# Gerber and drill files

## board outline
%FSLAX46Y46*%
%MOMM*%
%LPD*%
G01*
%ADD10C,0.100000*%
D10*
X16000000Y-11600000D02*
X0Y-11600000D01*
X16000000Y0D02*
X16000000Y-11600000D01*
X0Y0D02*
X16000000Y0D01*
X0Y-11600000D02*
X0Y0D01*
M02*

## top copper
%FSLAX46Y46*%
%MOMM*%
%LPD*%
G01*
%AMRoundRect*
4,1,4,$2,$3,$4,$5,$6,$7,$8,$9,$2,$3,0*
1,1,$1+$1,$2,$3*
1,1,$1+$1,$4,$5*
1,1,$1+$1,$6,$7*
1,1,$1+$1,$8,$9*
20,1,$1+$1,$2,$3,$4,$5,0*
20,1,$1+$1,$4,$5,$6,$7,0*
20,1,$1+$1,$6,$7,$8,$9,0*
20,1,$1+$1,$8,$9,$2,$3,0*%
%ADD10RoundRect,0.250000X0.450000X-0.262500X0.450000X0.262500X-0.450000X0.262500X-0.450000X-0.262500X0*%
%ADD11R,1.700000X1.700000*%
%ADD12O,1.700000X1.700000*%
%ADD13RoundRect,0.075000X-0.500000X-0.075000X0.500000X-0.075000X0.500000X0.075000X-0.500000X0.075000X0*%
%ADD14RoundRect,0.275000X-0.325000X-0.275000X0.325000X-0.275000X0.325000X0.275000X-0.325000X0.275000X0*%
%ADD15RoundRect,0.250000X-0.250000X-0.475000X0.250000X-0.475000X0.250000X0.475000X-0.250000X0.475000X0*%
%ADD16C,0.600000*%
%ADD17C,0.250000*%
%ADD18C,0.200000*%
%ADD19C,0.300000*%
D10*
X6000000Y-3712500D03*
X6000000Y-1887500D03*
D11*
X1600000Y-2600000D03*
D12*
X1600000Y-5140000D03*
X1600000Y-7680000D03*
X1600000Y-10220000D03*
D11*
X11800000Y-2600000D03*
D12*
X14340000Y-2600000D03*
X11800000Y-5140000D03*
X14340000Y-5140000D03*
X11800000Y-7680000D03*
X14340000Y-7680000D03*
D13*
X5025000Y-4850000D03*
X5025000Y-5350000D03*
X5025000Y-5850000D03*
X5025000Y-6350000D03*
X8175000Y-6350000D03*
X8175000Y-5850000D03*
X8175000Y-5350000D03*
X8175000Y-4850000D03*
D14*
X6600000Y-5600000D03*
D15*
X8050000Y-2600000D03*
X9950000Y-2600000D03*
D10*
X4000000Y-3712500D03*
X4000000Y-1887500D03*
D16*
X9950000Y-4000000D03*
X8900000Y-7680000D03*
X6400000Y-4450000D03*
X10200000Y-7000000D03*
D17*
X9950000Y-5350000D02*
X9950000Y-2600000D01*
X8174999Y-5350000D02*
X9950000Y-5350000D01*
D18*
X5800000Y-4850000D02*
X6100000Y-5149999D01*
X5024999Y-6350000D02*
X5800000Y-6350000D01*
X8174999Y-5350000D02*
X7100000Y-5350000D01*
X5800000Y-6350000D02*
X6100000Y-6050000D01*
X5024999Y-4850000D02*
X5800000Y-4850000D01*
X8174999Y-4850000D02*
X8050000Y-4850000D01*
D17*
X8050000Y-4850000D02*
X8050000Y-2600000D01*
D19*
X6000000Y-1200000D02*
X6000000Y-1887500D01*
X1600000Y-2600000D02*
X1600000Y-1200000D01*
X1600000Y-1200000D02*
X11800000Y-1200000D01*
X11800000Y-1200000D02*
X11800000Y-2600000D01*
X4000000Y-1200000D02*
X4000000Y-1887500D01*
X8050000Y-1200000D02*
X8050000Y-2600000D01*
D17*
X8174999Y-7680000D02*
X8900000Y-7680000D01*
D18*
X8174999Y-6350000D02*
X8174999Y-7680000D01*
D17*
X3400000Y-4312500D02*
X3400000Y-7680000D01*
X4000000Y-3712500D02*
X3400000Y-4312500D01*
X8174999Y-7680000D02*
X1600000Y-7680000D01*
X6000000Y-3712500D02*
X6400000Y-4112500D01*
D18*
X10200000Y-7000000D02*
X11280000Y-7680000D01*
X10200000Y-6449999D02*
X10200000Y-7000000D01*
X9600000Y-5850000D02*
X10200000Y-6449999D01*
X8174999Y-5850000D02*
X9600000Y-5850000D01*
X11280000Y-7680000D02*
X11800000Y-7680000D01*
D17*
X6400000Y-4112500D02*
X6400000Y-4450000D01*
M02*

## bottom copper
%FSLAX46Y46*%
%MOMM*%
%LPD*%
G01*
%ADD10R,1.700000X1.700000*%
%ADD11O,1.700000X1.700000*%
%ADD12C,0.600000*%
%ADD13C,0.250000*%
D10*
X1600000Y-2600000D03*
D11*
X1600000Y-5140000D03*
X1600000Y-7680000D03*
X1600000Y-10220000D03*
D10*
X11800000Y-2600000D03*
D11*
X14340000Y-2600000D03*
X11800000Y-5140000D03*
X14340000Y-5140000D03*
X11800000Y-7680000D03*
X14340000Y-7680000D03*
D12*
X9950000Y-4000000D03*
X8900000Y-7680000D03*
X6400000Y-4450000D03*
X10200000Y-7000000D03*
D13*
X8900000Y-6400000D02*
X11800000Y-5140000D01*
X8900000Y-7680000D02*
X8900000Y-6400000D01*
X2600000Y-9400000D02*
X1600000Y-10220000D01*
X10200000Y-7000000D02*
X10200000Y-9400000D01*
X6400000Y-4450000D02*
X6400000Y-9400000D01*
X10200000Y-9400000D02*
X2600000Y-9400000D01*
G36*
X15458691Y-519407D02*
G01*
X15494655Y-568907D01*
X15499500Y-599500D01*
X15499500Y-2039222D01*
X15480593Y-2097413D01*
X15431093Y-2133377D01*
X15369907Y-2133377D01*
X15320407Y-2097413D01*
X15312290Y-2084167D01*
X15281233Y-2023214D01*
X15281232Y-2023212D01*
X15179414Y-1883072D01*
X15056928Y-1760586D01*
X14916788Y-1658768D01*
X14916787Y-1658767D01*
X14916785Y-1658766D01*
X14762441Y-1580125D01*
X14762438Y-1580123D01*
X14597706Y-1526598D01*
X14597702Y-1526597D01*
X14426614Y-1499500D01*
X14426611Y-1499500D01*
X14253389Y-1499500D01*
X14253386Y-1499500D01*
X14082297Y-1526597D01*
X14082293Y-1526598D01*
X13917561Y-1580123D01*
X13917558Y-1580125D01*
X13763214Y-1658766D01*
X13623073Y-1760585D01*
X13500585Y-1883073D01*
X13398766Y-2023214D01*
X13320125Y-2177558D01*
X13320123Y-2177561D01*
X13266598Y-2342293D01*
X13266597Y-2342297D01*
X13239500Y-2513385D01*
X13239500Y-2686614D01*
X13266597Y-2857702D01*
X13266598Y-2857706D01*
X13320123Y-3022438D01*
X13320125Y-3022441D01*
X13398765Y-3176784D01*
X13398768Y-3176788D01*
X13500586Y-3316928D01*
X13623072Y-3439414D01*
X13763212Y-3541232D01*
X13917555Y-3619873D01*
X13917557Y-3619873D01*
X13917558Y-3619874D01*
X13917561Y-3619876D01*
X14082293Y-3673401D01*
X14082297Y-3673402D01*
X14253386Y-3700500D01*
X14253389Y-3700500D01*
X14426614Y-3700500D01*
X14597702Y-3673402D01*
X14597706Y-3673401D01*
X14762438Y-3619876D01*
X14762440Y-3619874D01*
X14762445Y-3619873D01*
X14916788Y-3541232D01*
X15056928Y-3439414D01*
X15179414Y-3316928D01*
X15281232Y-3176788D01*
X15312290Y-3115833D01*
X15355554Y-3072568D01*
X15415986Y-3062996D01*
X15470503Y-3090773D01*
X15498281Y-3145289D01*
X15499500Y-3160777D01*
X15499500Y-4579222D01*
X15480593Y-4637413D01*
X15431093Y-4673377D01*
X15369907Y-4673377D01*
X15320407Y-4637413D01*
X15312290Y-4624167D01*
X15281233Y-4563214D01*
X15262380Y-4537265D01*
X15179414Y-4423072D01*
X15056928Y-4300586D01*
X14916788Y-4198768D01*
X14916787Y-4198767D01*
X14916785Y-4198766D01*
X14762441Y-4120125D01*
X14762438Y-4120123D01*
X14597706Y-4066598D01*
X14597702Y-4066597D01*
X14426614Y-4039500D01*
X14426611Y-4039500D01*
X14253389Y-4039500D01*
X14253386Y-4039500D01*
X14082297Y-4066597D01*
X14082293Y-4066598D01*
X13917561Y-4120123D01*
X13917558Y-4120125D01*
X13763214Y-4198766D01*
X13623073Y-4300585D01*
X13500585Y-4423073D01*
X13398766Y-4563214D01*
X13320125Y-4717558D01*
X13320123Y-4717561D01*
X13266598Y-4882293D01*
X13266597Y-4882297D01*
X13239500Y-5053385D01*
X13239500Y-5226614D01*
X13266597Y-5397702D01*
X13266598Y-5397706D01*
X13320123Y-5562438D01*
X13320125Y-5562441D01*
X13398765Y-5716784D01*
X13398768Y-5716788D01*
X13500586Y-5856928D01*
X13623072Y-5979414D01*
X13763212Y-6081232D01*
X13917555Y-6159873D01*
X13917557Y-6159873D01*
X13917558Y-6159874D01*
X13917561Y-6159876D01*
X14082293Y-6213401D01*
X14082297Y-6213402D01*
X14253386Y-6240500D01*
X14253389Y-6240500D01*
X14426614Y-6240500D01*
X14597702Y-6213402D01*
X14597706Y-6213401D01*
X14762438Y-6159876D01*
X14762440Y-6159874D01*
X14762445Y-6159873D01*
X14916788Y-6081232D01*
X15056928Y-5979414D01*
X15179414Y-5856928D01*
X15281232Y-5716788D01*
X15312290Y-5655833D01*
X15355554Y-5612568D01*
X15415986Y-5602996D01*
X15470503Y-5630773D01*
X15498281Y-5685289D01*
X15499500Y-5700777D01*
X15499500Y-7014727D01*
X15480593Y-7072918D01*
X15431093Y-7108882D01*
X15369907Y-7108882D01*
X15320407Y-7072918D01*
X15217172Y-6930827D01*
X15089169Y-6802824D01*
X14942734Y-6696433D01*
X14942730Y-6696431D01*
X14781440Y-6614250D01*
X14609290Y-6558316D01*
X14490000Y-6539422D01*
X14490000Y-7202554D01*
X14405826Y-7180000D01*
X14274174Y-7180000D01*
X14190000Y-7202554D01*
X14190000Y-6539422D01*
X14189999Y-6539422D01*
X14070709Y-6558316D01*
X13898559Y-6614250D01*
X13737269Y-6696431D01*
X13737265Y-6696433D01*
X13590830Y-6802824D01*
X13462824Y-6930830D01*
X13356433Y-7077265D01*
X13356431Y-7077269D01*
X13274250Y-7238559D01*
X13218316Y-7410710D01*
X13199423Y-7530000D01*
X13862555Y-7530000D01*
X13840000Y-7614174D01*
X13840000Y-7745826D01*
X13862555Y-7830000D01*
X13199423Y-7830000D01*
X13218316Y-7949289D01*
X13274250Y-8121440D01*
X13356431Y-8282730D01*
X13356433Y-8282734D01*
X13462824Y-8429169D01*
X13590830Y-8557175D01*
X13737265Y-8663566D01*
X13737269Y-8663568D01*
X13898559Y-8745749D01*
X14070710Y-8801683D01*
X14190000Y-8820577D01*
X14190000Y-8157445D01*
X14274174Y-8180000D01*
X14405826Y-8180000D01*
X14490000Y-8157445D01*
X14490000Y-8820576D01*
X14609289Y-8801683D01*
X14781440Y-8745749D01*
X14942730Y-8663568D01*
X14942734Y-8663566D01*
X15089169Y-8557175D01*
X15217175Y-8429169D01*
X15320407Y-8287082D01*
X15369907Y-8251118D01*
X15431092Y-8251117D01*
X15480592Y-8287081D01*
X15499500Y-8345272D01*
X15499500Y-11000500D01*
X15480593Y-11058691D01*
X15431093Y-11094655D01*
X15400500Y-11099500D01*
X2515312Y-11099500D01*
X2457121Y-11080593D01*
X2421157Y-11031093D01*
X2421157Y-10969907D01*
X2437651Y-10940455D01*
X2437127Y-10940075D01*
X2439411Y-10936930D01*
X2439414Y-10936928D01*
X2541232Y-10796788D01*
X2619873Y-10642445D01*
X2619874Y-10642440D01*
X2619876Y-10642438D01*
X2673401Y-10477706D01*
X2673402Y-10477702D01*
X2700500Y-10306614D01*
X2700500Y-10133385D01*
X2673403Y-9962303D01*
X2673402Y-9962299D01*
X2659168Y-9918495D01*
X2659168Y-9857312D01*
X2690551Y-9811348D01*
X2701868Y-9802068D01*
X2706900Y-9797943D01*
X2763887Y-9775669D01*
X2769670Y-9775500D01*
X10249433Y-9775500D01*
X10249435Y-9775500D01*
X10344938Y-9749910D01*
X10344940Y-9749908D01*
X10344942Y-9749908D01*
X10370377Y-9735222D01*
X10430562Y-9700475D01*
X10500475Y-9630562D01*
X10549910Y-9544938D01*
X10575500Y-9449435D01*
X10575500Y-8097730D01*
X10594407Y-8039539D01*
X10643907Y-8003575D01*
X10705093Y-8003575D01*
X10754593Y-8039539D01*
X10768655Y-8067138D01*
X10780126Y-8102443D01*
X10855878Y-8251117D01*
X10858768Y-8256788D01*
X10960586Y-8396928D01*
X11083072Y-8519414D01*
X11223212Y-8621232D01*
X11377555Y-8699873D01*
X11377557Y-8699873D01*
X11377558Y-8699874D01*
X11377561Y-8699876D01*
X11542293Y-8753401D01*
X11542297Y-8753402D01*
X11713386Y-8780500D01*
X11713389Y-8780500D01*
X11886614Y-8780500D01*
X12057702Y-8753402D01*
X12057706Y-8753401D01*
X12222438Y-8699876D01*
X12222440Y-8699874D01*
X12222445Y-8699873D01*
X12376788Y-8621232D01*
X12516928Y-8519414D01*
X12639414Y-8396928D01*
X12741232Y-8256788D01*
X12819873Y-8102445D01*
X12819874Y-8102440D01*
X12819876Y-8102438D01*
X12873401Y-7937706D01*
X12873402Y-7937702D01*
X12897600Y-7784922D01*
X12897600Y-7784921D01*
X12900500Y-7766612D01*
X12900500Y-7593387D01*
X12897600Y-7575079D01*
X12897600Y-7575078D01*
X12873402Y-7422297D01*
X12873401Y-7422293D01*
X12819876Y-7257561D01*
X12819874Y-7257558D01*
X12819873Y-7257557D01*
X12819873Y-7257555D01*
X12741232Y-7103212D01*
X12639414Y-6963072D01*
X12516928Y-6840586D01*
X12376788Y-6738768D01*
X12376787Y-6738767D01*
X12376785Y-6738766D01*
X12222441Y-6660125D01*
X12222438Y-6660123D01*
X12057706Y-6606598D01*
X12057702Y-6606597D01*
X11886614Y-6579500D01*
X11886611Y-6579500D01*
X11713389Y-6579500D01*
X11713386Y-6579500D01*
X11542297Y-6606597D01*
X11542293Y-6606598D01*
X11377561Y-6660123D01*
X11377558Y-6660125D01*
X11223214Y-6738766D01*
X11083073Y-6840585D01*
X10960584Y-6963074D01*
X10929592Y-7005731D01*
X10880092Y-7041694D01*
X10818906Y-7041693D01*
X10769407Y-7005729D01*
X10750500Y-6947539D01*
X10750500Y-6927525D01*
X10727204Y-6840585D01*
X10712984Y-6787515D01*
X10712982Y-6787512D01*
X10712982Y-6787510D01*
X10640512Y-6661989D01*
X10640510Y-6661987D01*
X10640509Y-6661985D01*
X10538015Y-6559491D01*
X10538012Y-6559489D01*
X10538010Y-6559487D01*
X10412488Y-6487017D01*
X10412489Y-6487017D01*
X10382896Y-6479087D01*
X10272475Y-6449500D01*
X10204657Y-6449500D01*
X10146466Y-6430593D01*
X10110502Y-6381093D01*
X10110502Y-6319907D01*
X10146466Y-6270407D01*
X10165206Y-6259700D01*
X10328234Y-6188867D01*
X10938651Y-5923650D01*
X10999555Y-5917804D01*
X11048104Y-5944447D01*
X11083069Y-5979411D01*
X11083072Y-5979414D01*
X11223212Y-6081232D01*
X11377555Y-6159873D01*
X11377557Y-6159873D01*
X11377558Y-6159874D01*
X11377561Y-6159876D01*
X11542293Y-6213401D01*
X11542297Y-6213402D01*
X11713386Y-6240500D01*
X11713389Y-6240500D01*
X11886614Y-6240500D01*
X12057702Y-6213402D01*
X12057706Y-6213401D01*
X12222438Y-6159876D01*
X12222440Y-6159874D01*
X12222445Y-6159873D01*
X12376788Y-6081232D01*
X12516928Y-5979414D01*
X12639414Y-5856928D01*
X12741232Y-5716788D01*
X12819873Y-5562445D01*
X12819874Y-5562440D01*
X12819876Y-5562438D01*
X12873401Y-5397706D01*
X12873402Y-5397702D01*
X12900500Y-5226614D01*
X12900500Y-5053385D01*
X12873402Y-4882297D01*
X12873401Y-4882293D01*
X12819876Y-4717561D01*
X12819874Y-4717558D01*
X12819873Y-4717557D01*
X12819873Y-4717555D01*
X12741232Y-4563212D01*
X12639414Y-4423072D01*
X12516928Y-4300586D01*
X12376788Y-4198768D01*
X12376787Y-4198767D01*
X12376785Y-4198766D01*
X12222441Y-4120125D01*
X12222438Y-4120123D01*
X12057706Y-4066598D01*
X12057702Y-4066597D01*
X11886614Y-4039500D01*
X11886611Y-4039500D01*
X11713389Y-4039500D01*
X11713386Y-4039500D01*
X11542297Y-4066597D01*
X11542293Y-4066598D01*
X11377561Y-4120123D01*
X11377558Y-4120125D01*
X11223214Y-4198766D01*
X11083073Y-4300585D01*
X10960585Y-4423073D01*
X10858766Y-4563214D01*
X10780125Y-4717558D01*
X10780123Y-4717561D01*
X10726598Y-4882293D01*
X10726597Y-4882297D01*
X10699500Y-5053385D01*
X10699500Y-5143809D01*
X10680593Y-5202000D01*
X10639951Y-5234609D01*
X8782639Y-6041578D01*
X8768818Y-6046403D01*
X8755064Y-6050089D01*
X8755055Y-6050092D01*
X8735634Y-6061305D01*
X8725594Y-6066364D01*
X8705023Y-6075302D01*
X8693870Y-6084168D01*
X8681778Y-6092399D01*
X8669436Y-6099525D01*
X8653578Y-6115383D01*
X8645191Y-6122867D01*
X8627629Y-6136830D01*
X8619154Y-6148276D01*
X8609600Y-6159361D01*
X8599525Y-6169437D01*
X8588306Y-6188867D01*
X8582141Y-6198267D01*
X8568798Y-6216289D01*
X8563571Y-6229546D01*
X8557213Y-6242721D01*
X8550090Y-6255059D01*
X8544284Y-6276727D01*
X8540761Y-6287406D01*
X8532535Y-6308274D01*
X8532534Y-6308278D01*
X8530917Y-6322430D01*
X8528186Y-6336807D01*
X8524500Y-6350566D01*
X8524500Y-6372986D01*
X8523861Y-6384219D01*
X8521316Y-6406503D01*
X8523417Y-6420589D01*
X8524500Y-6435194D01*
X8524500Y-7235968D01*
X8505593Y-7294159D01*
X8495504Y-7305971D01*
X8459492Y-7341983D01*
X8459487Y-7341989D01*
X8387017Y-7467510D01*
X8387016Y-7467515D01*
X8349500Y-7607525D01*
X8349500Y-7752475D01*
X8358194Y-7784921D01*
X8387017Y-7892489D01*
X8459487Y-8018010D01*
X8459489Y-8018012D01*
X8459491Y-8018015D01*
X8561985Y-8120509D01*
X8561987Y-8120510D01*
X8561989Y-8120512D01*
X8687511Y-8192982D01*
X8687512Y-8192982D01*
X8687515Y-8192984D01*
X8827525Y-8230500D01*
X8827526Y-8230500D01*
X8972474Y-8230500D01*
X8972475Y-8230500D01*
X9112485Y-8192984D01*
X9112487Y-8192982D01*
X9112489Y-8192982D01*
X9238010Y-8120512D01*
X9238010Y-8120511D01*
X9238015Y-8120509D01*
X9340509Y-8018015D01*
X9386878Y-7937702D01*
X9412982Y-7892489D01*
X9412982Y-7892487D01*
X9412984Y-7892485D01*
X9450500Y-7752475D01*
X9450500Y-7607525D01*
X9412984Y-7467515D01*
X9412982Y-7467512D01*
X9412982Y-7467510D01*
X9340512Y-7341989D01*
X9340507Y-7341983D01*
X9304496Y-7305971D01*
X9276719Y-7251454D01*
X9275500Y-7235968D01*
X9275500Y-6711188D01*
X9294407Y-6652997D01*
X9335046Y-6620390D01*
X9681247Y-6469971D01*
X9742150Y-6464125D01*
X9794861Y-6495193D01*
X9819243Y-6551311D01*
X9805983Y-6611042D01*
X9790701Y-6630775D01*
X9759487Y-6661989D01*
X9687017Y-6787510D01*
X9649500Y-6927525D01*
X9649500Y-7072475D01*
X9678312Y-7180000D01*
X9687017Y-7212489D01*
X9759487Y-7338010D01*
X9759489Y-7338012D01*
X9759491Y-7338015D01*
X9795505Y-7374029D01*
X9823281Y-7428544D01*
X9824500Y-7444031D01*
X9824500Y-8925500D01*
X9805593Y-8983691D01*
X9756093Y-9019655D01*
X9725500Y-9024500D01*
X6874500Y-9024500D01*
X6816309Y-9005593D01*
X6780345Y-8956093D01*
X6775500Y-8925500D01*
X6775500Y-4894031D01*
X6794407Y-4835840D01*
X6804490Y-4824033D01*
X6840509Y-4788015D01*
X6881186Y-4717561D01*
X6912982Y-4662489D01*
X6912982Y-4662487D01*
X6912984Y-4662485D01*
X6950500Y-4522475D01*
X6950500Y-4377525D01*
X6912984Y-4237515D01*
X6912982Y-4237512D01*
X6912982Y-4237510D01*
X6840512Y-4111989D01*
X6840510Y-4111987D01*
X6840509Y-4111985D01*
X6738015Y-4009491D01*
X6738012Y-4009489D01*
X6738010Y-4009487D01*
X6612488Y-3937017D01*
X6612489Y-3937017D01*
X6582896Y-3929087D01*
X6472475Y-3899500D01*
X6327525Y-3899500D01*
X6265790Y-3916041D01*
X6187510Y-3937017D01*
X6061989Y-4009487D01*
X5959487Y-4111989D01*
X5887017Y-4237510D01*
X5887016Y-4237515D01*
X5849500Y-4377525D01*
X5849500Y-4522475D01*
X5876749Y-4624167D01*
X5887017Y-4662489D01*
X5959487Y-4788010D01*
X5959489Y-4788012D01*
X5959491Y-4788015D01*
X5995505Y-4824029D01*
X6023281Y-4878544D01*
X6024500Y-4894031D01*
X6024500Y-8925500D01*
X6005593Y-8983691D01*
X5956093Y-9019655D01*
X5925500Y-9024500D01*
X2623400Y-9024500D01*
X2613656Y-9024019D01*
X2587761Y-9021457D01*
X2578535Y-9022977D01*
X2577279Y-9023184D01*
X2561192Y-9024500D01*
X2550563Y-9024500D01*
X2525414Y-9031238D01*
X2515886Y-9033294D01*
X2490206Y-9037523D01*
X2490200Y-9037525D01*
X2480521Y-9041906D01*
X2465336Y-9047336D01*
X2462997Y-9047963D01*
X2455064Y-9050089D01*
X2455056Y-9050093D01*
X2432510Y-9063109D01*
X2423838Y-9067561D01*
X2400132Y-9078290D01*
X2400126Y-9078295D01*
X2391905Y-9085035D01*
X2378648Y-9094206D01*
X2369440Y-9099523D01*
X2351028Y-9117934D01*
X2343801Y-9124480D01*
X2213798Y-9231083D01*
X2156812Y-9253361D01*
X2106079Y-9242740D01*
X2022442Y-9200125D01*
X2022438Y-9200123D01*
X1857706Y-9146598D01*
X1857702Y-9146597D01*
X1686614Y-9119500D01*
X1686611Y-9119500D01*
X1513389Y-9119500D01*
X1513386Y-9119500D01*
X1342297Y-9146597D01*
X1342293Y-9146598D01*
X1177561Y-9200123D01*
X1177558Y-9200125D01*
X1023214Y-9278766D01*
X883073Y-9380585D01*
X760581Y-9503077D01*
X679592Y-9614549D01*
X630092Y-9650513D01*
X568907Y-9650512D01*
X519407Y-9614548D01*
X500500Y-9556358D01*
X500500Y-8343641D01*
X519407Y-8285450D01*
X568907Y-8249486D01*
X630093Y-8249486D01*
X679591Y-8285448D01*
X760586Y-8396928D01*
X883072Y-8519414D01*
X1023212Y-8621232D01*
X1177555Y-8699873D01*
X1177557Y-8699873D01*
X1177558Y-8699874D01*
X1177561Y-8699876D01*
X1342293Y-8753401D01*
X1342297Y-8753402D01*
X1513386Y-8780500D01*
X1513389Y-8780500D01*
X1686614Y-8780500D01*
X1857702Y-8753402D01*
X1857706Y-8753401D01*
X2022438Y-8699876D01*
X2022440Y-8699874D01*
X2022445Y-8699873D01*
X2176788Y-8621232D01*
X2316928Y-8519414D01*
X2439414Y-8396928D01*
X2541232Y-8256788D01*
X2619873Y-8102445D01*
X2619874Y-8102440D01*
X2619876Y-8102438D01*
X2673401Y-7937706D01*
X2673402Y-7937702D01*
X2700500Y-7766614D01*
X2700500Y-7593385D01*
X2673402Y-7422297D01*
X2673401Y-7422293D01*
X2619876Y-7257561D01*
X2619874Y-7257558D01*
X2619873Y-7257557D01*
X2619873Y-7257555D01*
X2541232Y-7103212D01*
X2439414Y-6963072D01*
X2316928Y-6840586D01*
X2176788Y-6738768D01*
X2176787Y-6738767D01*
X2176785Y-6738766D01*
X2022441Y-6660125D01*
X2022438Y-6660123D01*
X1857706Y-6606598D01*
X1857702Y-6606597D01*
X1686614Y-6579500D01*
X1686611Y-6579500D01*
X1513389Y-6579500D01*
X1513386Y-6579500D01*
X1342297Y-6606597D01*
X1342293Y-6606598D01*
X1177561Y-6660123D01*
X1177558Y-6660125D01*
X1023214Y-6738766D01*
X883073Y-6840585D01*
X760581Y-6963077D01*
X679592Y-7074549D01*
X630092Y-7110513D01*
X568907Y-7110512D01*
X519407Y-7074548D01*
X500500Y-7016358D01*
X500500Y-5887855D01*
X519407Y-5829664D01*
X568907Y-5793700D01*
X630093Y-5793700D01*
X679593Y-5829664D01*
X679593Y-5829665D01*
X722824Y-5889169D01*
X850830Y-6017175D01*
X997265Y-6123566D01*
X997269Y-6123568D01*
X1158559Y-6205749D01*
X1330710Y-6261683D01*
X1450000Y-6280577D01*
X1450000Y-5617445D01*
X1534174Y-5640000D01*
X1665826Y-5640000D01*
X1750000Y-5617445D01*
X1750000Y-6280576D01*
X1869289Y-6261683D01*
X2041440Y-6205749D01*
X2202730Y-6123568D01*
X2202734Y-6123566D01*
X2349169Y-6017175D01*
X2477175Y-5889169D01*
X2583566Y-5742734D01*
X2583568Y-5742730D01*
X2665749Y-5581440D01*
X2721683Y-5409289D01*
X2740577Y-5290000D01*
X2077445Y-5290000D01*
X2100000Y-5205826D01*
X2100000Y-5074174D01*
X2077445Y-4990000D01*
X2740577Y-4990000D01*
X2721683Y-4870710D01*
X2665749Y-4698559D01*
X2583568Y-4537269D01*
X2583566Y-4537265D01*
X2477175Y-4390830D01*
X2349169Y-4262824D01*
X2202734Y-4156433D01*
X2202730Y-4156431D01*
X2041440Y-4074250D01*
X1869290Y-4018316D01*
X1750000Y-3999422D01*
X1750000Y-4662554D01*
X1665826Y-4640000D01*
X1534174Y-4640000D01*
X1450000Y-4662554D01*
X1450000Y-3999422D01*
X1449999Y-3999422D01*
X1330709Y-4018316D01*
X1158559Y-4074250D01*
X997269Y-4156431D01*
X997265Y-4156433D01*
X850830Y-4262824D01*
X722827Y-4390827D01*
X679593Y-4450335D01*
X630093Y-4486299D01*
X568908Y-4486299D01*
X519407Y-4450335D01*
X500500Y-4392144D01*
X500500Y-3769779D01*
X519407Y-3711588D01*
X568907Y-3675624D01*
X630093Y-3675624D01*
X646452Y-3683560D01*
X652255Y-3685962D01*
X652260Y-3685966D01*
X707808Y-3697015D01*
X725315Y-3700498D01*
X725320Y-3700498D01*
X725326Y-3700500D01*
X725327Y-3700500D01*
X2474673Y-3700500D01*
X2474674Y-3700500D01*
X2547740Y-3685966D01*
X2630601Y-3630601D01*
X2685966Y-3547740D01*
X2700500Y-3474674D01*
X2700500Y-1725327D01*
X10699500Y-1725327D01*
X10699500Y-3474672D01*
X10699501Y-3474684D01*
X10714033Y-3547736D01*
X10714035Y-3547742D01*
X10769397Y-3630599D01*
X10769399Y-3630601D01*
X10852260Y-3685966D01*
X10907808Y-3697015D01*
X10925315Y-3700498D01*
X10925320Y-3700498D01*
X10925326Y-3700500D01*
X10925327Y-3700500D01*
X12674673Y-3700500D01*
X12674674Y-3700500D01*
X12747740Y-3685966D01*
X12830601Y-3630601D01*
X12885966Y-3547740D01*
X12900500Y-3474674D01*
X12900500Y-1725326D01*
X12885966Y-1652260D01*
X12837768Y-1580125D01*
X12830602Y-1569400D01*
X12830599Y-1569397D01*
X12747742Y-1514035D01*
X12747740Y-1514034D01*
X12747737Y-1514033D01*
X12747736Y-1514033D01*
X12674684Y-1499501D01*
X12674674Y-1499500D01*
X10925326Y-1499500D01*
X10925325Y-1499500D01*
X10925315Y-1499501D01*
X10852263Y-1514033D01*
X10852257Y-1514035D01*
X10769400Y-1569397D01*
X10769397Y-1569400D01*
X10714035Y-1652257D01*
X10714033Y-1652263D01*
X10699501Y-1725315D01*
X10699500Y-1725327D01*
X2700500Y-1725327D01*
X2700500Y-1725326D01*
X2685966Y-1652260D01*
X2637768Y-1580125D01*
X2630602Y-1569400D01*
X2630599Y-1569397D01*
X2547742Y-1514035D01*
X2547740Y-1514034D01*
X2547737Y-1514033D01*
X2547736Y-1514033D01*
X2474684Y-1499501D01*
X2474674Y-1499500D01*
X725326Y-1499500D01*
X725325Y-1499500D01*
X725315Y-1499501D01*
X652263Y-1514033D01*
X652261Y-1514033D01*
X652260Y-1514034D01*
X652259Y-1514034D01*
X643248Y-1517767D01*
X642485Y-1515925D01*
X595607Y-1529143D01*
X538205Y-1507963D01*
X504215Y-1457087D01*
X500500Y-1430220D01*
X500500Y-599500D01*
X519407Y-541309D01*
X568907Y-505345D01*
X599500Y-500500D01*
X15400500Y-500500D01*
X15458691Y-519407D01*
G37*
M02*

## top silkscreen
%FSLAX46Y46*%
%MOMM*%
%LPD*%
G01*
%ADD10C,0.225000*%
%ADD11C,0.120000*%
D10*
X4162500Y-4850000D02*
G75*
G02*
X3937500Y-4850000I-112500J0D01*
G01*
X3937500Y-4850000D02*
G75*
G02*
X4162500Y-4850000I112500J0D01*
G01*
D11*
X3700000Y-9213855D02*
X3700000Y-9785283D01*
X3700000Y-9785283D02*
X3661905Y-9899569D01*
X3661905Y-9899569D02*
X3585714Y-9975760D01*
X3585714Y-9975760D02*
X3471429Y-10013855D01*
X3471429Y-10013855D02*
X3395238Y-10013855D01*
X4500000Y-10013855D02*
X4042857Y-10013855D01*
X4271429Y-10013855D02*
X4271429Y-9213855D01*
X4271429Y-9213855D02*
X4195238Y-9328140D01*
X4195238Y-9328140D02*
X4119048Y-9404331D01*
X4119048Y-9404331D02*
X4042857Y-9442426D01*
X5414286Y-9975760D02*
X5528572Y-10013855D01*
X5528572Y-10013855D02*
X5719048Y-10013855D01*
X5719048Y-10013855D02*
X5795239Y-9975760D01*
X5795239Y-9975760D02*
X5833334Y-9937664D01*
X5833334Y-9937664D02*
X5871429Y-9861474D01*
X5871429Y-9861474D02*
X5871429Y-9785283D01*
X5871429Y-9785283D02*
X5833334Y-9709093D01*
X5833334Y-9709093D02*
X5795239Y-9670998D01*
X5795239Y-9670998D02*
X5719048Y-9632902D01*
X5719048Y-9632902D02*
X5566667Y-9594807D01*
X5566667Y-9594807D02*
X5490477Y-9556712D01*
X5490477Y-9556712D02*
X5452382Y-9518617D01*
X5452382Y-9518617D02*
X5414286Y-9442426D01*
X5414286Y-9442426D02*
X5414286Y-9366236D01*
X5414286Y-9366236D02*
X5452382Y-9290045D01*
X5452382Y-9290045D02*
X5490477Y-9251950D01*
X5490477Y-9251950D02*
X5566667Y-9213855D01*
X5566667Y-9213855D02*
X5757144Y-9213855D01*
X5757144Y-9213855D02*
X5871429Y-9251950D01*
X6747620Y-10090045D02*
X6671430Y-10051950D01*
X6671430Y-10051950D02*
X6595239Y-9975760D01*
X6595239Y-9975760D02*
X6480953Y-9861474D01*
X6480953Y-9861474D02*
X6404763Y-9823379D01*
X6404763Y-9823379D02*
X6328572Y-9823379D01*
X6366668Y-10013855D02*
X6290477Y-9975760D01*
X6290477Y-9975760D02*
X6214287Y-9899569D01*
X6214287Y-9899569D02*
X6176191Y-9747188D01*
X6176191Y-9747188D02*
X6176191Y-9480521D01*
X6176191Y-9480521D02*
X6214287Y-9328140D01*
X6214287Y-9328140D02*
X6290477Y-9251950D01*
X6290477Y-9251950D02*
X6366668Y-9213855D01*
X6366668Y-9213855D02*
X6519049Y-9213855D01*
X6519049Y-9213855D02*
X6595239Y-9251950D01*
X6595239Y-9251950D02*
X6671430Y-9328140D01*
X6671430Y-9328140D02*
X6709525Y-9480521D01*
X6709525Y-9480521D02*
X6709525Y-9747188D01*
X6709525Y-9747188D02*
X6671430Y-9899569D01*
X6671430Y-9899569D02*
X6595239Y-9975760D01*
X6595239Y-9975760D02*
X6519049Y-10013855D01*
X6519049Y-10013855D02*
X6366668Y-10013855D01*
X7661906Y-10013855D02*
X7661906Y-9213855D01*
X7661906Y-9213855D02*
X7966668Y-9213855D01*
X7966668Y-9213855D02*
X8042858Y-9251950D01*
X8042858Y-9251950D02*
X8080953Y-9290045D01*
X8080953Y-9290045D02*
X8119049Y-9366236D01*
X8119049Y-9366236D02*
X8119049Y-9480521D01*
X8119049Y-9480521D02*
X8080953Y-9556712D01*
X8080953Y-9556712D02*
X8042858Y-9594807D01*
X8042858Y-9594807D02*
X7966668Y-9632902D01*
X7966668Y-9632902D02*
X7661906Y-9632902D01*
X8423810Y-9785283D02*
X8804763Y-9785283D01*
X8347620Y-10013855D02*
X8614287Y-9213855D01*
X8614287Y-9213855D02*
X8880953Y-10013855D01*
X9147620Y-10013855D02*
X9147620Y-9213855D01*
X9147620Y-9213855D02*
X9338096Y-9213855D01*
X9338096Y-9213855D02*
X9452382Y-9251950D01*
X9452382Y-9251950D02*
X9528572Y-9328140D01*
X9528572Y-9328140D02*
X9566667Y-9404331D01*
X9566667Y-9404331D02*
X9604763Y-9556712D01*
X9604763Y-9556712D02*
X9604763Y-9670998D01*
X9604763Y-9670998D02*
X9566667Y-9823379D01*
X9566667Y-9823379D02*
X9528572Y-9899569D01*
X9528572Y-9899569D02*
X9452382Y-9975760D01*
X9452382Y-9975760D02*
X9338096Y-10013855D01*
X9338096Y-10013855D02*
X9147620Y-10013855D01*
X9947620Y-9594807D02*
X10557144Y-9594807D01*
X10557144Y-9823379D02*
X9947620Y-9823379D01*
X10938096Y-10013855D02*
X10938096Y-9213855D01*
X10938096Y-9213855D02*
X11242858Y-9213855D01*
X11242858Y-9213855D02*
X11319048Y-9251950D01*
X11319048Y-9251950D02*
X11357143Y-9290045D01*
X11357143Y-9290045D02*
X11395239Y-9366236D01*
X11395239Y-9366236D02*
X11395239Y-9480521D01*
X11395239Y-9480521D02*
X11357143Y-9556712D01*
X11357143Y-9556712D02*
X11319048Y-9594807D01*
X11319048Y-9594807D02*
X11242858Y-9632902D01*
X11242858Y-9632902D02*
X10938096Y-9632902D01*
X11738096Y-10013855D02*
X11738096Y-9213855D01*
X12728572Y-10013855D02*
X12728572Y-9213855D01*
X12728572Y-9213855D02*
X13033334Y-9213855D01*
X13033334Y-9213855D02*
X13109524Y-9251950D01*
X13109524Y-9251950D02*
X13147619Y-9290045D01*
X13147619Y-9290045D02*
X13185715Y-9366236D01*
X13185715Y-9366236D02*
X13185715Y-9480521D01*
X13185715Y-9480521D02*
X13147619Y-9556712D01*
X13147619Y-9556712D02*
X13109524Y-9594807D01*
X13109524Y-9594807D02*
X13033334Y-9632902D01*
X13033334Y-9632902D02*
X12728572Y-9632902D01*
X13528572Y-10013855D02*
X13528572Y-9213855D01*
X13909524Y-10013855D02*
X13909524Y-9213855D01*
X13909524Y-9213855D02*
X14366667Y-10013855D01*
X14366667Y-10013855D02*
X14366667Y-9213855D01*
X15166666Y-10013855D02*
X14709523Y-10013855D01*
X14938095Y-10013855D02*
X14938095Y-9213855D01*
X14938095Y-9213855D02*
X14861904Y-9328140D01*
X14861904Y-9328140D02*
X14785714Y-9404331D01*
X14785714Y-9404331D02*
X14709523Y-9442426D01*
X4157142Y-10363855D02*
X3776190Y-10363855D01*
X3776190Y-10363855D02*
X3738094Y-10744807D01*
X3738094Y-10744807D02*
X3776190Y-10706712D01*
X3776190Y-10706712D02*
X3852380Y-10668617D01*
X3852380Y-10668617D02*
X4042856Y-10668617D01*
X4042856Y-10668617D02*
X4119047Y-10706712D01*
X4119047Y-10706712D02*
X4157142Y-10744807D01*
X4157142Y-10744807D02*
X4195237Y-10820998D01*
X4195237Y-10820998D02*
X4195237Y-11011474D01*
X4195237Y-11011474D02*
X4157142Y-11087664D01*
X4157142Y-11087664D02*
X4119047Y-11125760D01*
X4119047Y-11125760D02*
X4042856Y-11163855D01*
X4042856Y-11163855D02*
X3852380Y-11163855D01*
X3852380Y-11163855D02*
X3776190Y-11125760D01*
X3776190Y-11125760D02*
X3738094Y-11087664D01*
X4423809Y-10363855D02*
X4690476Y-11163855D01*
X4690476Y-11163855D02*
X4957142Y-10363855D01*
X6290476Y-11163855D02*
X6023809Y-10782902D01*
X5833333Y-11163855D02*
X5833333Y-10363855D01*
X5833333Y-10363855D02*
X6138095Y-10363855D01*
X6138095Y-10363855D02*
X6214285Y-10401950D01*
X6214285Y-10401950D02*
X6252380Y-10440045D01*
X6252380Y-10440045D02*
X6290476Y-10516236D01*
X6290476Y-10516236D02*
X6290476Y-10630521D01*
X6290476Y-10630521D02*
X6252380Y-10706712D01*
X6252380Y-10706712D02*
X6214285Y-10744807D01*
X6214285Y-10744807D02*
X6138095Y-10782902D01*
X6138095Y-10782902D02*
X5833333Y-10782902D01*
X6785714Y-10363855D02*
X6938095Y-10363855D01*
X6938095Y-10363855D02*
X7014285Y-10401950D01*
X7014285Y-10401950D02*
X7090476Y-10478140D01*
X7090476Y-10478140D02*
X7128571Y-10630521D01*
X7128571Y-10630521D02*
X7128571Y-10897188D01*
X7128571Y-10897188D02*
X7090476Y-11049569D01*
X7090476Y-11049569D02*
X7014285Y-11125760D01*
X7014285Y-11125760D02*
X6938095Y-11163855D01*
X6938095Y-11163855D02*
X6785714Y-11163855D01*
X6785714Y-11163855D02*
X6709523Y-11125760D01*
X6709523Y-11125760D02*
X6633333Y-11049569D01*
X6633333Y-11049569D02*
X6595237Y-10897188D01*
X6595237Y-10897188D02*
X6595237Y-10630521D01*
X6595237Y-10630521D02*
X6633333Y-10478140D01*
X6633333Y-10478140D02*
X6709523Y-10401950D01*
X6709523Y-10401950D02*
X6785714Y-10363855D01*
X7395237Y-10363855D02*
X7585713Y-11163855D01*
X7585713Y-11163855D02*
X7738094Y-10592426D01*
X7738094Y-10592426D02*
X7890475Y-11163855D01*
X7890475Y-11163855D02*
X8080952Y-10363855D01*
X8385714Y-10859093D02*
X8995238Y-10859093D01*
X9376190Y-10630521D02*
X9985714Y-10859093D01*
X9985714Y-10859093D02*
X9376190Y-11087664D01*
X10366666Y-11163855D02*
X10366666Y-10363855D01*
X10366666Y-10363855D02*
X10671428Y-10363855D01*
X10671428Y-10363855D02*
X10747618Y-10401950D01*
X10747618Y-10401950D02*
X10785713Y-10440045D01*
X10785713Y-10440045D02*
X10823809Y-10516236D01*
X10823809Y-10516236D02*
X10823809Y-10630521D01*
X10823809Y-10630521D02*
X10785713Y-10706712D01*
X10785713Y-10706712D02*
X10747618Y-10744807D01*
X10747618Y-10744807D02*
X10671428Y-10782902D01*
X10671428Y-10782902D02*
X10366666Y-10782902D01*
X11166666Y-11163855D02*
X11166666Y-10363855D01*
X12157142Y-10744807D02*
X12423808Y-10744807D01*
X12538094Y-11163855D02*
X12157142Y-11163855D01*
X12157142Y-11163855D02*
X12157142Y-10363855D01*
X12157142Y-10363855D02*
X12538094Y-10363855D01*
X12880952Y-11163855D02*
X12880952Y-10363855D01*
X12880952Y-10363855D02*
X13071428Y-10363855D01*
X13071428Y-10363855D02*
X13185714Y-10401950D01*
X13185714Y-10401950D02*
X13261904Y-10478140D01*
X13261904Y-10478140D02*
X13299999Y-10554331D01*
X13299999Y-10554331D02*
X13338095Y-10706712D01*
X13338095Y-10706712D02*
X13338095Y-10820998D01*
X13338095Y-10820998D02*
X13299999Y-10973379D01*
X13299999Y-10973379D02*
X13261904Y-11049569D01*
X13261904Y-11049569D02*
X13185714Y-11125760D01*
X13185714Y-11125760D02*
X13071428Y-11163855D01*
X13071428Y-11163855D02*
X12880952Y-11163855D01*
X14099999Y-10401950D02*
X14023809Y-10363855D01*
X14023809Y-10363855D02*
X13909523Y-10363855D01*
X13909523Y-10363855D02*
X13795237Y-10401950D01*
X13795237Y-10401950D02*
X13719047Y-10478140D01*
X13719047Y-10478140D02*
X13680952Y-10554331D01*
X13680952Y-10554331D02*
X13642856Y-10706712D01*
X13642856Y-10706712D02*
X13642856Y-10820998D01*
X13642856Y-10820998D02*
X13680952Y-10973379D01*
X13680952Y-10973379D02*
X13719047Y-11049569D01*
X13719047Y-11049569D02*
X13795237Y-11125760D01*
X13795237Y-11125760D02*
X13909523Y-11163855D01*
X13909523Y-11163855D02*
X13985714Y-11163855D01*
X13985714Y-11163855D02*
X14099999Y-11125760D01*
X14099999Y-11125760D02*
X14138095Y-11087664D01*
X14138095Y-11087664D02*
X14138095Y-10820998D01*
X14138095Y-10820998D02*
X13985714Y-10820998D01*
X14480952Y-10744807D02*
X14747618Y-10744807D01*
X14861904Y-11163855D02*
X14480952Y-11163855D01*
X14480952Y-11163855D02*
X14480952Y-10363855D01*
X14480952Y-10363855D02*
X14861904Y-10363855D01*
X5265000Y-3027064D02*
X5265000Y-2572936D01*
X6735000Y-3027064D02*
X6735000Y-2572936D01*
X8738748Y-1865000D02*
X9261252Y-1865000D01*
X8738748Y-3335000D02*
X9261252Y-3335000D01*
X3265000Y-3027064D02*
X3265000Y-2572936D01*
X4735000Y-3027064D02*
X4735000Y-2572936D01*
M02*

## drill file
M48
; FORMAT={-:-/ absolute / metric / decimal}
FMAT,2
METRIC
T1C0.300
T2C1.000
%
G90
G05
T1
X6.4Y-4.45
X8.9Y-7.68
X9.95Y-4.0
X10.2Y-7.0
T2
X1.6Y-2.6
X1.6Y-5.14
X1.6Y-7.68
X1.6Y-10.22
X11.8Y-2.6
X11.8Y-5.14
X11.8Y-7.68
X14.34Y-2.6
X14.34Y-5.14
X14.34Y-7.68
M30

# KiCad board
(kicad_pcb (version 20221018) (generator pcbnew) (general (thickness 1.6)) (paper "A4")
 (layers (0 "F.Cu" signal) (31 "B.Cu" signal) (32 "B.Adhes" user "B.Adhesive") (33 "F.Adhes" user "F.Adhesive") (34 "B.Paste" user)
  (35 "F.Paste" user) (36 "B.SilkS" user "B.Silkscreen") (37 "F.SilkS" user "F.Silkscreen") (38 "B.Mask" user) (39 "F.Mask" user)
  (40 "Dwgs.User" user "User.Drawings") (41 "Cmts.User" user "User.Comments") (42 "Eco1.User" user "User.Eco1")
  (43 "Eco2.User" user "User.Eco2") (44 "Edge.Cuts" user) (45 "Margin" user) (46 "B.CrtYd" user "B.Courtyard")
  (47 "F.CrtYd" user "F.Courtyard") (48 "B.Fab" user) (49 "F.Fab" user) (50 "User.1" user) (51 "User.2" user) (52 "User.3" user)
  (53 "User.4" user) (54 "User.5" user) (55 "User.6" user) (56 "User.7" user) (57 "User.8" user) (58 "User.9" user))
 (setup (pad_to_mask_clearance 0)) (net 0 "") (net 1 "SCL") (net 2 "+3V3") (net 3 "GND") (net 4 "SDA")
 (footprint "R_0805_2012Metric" (layer "F.Cu") (at 6 2.8 90)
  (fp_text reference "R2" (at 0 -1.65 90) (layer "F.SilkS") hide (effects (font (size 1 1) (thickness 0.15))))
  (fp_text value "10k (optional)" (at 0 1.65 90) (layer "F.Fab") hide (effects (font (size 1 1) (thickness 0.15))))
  (fp_line (start -0.227064 -0.735) (end 0.227064 -0.735) (stroke (width 0.12) (type solid)) (layer "F.SilkS"))
  (fp_line (start -0.227064 0.735) (end 0.227064 0.735) (stroke (width 0.12) (type solid)) (layer "F.SilkS"))
  (pad "1" smd roundrect (at -0.9125 0 90) (size 1.025 1.4) (layers "F.Cu" "F.Paste" "F.Mask") (roundrect_rratio 0.243902) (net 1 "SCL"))
  (pad "2" smd roundrect (at 0.9125 0 90) (size 1.025 1.4) (layers "F.Cu" "F.Paste" "F.Mask") (roundrect_rratio 0.243902) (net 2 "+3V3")))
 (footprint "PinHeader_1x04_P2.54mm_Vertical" (layer "F.Cu") (at 1.6 2.6)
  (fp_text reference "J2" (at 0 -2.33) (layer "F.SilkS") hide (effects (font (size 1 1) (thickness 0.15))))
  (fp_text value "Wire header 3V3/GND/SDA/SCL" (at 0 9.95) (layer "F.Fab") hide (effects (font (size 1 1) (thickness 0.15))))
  (pad "1" thru_hole rect (at 0 0) (size 1.7 1.7) (drill 1) (layers "*.Cu" "*.Mask") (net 2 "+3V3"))
  (pad "2" thru_hole oval (at 0 2.54) (size 1.7 1.7) (drill 1) (layers "*.Cu" "*.Mask") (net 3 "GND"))
  (pad "3" thru_hole oval (at 0 5.08) (size 1.7 1.7) (drill 1) (layers "*.Cu" "*.Mask") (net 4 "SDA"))
  (pad "4" thru_hole oval (at 0 7.62) (size 1.7 1.7) (drill 1) (layers "*.Cu" "*.Mask") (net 1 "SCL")))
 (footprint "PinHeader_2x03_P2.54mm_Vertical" (layer "F.Cu") (at 11.8 2.6)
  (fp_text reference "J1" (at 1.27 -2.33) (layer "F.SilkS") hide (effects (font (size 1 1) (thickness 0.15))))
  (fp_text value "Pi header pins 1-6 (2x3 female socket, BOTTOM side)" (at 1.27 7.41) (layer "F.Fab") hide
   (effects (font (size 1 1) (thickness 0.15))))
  (pad "1" thru_hole rect (at 0 0) (size 1.7 1.7) (drill 1) (layers "*.Cu" "*.Mask") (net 2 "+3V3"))
  (pad "2" thru_hole oval (at 2.54 0) (size 1.7 1.7) (drill 1) (layers "*.Cu" "*.Mask"))
  (pad "3" thru_hole oval (at 0 2.54) (size 1.7 1.7) (drill 1) (layers "*.Cu" "*.Mask") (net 4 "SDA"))
  (pad "4" thru_hole oval (at 2.54 2.54) (size 1.7 1.7) (drill 1) (layers "*.Cu" "*.Mask"))
  (pad "5" thru_hole oval (at 0 5.08) (size 1.7 1.7) (drill 1) (layers "*.Cu" "*.Mask") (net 1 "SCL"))
  (pad "6" thru_hole oval (at 2.54 5.08) (size 1.7 1.7) (drill 1) (layers "*.Cu" "*.Mask") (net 3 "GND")))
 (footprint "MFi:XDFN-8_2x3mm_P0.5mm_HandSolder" (layer "F.Cu") (at 6.6 5.6)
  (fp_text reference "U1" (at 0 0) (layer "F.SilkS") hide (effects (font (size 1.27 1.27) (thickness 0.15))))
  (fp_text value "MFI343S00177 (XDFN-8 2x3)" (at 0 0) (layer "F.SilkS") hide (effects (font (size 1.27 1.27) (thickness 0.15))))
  (pad "1" smd roundrect (at -1.575 -0.75) (size 1.15 0.3) (layers "F.Cu" "F.Paste" "F.Mask") (roundrect_rratio 0.25) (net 3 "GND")
   (thermal_bridge_angle 45))
  (pad "2" smd roundrect (at -1.575 -0.25) (size 1.15 0.3) (layers "F.Cu" "F.Paste" "F.Mask") (roundrect_rratio 0.25)
   (thermal_bridge_angle 45))
  (pad "3" smd roundrect (at -1.575 0.25) (size 1.15 0.3) (layers "F.Cu" "F.Paste" "F.Mask") (roundrect_rratio 0.25)
   (thermal_bridge_angle 45))
  (pad "4" smd roundrect (at -1.575 0.75) (size 1.15 0.3) (layers "F.Cu" "F.Paste" "F.Mask") (roundrect_rratio 0.25) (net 3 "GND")
   (thermal_bridge_angle 45))
  (pad "5" smd roundrect (at 1.575 0.75) (size 1.15 0.3) (layers "F.Cu" "F.Paste" "F.Mask") (roundrect_rratio 0.25) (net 4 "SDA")
   (thermal_bridge_angle 45))
  (pad "6" smd roundrect (at 1.575 0.25) (size 1.15 0.3) (layers "F.Cu" "F.Paste" "F.Mask") (roundrect_rratio 0.25) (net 1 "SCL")
   (thermal_bridge_angle 45))
  (pad "7" smd roundrect (at 1.575 -0.25) (size 1.15 0.3) (layers "F.Cu" "F.Paste" "F.Mask") (roundrect_rratio 0.25) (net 3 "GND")
   (thermal_bridge_angle 45))
  (pad "8" smd roundrect (at 1.575 -0.75) (size 1.15 0.3) (layers "F.Cu" "F.Paste" "F.Mask") (roundrect_rratio 0.25) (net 2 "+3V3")
   (thermal_bridge_angle 45))
  (pad "9" smd roundrect (at 0 0) (size 1.2 1.1) (layers "F.Cu" "F.Paste" "F.Mask") (roundrect_rratio 0.25) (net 3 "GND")
   (thermal_bridge_angle 45)))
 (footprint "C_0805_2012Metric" (layer "F.Cu") (at 9 2.6)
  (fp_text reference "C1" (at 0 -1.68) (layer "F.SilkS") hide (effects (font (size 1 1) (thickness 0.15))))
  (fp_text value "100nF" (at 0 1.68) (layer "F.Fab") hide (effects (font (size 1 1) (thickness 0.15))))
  (fp_line (start -0.261252 -0.735) (end 0.261252 -0.735) (stroke (width 0.12) (type solid)) (layer "F.SilkS"))
  (fp_line (start -0.261252 0.735) (end 0.261252 0.735) (stroke (width 0.12) (type solid)) (layer "F.SilkS"))
  (pad "1" smd roundrect (at -0.95 0) (size 1 1.45) (layers "F.Cu" "F.Paste" "F.Mask") (roundrect_rratio 0.25) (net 2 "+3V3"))
  (pad "2" smd roundrect (at 0.95 0) (size 1 1.45) (layers "F.Cu" "F.Paste" "F.Mask") (roundrect_rratio 0.25) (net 3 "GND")))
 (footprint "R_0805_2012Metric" (layer "F.Cu") (at 4 2.8 90)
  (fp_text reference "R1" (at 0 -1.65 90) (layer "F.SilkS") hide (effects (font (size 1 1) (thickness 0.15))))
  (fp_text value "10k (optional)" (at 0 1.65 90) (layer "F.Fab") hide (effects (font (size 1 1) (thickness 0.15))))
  (fp_line (start -0.227064 -0.735) (end 0.227064 -0.735) (stroke (width 0.12) (type solid)) (layer "F.SilkS"))
  (fp_line (start -0.227064 0.735) (end 0.227064 0.735) (stroke (width 0.12) (type solid)) (layer "F.SilkS"))
  (pad "1" smd roundrect (at -0.9125 0 90) (size 1.025 1.4) (layers "F.Cu" "F.Paste" "F.Mask") (roundrect_rratio 0.243902) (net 4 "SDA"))
  (pad "2" smd roundrect (at 0.9125 0 90) (size 1.025 1.4) (layers "F.Cu" "F.Paste" "F.Mask") (roundrect_rratio 0.243902) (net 2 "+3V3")))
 (gr_circle (center 4.05 4.85) (end 4.2 4.85) (stroke (width 0.15) (type default)) (fill solid) (layer "F.SilkS"))
 (gr_line (start 16 11.6) (end 0 11.6) (stroke (width 0.1) (type default)) (layer "Edge.Cuts"))
 (gr_line (start 16 0) (end 16 11.6) (stroke (width 0.1) (type default)) (layer "Edge.Cuts"))
 (gr_line (start 0 0) (end 16 0) (stroke (width 0.1) (type default)) (layer "Edge.Cuts"))
 (gr_line (start 0 11.6) (end 0 0) (stroke (width 0.1) (type default)) (layer "Edge.Cuts"))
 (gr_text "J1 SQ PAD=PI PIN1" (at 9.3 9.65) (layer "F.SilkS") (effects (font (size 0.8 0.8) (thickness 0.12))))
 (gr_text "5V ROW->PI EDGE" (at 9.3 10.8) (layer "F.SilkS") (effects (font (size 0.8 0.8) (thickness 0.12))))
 (segment (start 9.95 5.35) (end 9.95 2.6) (width 0.25) (layer "F.Cu") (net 3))
 (segment (start 8.174999 5.35) (end 9.95 5.35) (width 0.25) (layer "F.Cu") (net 3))
 (segment (start 5.8 4.85) (end 6.1 5.149999) (width 0.2) (layer "F.Cu") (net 3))
 (segment (start 5.024999 6.35) (end 5.8 6.35) (width 0.2) (layer "F.Cu") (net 3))
 (segment (start 8.174999 5.35) (end 7.1 5.35) (width 0.2) (layer "F.Cu") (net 3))
 (segment (start 5.8 6.35) (end 6.1 6.05) (width 0.2) (layer "F.Cu") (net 3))
 (segment (start 5.024999 4.85) (end 5.8 4.85) (width 0.2) (layer "F.Cu") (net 3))
 (via (at 9.95 4) (size 0.6) (drill 0.3) (layers "F.Cu" "B.Cu") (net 3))
 (segment (start 8.174999 4.85) (end 8.05 4.85) (width 0.2) (layer "F.Cu") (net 2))
 (segment (start 8.05 4.85) (end 8.05 2.6) (width 0.25) (layer "F.Cu") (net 2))
 (segment (start 6 1.2) (end 6 1.8875) (width 0.3) (layer "F.Cu") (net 2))
 (segment (start 1.6 2.6) (end 1.6 1.2) (width 0.3) (layer "F.Cu") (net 2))
 (segment (start 1.6 1.2) (end 11.8 1.2) (width 0.3) (layer "F.Cu") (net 2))
 (segment (start 11.8 1.2) (end 11.8 2.6) (width 0.3) (layer "F.Cu") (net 2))
 (segment (start 4 1.2) (end 4 1.8875) (width 0.3) (layer "F.Cu") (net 2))
 (segment (start 8.05 1.2) (end 8.05 2.6) (width 0.3) (layer "F.Cu") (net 2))
 (segment (start 8.174999 7.68) (end 8.9 7.68) (width 0.25) (layer "F.Cu") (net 4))
 (segment (start 8.174999 6.35) (end 8.174999 7.68) (width 0.2) (layer "F.Cu") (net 4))
 (segment (start 3.4 4.3125) (end 3.4 7.68) (width 0.25) (layer "F.Cu") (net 4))
 (segment (start 4 3.7125) (end 3.4 4.3125) (width 0.25) (layer "F.Cu") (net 4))
 (segment (start 8.174999 7.68) (end 1.6 7.68) (width 0.25) (layer "F.Cu") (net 4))
 (via (at 8.9 7.68) (size 0.6) (drill 0.3) (layers "F.Cu" "B.Cu") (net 4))
 (segment (start 8.9 6.4) (end 11.8 5.14) (width 0.25) (layer "B.Cu") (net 4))
 (segment (start 8.9 7.68) (end 8.9 6.4) (width 0.25) (layer "B.Cu") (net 4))
 (segment (start 6 3.7125) (end 6.4 4.1125) (width 0.25) (layer "F.Cu") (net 1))
 (segment (start 10.2 7) (end 11.28 7.68) (width 0.2) (layer "F.Cu") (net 1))
 (segment (start 10.2 6.449999) (end 10.2 7) (width 0.2) (layer "F.Cu") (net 1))
 (segment (start 9.6 5.85) (end 10.2 6.449999) (width 0.2) (layer "F.Cu") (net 1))
 (segment (start 8.174999 5.85) (end 9.6 5.85) (width 0.2) (layer "F.Cu") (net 1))
 (segment (start 11.28 7.68) (end 11.8 7.68) (width 0.2) (layer "F.Cu") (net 1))
 (segment (start 6.4 4.1125) (end 6.4 4.45) (width 0.25) (layer "F.Cu") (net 1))
 (via (at 6.4 4.45) (size 0.6) (drill 0.3) (layers "F.Cu" "B.Cu") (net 1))
 (via (at 10.2 7) (size 0.6) (drill 0.3) (layers "F.Cu" "B.Cu") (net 1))
 (segment (start 2.6 9.4) (end 1.6 10.22) (width 0.25) (layer "B.Cu") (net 1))
 (segment (start 10.2 7) (end 10.2 9.4) (width 0.25) (layer "B.Cu") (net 1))
 (segment (start 6.4 4.45) (end 6.4 9.4) (width 0.25) (layer "B.Cu") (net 1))
 (segment (start 10.2 9.4) (end 2.6 9.4) (width 0.25) (layer "B.Cu") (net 1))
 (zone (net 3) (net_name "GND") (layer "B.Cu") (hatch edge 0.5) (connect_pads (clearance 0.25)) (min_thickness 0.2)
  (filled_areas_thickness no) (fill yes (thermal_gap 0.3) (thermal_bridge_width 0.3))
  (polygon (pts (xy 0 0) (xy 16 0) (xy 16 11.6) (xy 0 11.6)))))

